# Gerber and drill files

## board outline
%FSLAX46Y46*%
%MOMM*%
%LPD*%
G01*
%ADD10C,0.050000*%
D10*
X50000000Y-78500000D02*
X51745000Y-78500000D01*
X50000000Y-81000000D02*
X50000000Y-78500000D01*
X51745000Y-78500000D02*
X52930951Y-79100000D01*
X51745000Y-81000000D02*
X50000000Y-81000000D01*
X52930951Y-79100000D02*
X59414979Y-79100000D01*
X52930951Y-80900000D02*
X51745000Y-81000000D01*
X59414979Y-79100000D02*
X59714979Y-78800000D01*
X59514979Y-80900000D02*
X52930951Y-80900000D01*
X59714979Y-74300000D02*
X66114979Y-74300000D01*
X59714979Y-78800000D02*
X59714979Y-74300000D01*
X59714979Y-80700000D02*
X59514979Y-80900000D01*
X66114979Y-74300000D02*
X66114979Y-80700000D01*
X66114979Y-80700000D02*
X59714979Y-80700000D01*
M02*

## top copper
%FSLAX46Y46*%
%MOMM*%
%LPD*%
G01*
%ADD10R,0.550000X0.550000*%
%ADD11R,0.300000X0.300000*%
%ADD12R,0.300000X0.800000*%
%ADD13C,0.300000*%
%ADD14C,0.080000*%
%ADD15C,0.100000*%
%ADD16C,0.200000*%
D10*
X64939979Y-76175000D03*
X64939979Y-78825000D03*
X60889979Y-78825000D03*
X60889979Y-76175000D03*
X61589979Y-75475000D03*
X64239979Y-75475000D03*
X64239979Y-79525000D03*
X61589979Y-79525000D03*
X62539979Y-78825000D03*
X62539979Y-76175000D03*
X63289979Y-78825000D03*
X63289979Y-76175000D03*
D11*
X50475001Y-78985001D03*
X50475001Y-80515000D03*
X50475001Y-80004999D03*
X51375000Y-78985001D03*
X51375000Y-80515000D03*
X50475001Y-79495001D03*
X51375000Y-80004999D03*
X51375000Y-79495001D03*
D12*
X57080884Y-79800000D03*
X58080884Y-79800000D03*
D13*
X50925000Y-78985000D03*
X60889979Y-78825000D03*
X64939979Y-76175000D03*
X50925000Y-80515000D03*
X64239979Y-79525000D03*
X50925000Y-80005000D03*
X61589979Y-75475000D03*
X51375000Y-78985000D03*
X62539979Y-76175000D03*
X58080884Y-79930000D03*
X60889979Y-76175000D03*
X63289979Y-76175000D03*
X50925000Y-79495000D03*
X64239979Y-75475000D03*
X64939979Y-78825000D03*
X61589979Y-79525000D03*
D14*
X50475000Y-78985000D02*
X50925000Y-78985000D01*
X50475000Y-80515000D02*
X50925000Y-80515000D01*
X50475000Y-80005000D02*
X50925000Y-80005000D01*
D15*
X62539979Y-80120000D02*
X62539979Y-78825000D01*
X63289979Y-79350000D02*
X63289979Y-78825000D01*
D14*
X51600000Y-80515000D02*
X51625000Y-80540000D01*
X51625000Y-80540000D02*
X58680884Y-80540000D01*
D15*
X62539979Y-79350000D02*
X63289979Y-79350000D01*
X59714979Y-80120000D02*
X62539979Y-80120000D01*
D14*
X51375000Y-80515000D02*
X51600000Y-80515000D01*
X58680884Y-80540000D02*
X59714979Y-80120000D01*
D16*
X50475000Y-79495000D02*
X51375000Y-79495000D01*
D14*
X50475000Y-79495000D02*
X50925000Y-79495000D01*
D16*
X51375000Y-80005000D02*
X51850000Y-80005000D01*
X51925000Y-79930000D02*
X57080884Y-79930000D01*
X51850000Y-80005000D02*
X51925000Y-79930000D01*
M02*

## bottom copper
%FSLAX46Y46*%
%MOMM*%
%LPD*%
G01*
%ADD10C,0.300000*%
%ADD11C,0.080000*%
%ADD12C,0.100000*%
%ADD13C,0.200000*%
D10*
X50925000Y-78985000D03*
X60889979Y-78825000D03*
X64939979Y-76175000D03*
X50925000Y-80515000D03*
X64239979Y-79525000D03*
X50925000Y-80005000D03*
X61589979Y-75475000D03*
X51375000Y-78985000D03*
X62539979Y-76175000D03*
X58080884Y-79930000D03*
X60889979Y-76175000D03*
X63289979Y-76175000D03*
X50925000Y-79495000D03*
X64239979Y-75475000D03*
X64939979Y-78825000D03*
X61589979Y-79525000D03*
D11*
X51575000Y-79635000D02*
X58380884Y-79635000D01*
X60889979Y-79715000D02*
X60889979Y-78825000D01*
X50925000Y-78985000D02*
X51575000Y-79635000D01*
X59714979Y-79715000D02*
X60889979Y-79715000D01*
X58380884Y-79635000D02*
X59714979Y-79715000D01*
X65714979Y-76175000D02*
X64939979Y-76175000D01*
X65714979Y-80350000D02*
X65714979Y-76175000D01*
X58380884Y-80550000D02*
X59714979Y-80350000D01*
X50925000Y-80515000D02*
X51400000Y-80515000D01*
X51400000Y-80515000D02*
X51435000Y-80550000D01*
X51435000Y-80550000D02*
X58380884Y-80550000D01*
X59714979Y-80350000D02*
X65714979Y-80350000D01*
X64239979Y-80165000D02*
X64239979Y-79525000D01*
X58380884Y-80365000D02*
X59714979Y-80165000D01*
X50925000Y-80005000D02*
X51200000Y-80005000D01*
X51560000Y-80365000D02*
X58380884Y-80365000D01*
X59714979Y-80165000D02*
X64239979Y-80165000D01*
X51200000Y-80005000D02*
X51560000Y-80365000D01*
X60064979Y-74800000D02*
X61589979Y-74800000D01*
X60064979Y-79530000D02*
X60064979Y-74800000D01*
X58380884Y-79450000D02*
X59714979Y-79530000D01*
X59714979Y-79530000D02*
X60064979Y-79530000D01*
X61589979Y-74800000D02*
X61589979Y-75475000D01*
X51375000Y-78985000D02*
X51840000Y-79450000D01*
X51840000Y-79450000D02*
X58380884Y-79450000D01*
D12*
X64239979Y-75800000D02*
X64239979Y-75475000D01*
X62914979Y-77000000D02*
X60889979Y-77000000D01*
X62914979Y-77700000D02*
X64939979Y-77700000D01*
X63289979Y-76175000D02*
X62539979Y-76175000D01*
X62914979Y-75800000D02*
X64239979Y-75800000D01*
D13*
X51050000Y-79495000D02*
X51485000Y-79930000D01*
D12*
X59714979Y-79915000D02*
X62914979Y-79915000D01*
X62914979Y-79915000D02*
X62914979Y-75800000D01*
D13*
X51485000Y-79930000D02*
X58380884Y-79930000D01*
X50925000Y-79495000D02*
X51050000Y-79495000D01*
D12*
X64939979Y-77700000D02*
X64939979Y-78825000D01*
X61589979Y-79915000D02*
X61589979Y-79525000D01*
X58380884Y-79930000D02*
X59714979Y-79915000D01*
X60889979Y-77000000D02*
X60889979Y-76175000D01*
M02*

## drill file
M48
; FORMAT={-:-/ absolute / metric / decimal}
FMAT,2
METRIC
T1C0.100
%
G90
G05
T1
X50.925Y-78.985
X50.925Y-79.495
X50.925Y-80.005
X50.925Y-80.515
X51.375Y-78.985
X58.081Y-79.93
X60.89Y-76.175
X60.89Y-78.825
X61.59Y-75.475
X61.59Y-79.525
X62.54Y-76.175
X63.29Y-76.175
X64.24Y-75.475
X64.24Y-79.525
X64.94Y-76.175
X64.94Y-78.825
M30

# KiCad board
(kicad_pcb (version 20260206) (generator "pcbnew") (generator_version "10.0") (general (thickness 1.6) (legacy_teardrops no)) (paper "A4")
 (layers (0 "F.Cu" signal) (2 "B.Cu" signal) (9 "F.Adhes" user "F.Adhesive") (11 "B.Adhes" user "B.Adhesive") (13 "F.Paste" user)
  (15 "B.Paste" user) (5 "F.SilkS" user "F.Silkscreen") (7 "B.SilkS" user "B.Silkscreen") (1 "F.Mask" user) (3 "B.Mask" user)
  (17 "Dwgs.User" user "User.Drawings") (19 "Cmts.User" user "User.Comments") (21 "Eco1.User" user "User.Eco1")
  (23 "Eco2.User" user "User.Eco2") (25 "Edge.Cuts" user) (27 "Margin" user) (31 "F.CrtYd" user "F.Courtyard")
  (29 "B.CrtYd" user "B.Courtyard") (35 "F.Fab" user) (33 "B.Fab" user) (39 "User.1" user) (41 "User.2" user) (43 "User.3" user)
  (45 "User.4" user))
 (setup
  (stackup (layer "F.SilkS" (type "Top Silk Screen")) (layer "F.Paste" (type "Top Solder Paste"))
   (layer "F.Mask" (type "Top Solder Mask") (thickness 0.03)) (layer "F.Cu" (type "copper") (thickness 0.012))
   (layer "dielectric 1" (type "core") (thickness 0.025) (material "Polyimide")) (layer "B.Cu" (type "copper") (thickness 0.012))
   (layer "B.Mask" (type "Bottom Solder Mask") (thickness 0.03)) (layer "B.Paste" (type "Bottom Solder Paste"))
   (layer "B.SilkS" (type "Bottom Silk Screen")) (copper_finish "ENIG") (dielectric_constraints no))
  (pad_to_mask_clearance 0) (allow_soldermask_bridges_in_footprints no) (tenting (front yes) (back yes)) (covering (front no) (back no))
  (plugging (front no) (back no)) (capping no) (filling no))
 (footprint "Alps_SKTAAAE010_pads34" (layer "F.Cu") (at 62.914979 79.9 180)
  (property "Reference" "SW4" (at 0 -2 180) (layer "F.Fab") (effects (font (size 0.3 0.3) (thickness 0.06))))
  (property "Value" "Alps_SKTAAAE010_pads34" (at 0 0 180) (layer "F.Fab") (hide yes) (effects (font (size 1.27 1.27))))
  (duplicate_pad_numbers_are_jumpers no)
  (pad "3" smd rect (at -1.325 0.375 180) (size 0.55 0.55) (layers "F.Cu" "F.Mask" "F.Paste") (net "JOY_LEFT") (solder_mask_margin 0.05)
   (thermal_bridge_angle 45))
  (pad "4" smd rect (at 1.325 0.375 180) (size 0.55 0.55) (layers "F.Cu" "F.Mask" "F.Paste") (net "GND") (solder_mask_margin 0.05)
   (thermal_bridge_angle 45)))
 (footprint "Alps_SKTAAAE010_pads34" (layer "F.Cu") (at 62.914979 75.1)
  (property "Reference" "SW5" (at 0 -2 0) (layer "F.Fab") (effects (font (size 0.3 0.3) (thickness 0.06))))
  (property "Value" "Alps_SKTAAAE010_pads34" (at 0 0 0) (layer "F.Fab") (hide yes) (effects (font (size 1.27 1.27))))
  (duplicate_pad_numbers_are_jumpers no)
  (pad "3" smd rect (at -1.325 0.375) (size 0.55 0.55) (layers "F.Cu" "F.Mask" "F.Paste") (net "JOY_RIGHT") (solder_mask_margin 0.05)
   (thermal_bridge_angle 45))
  (pad "4" smd rect (at 1.325 0.375) (size 0.55 0.55) (layers "F.Cu" "F.Mask" "F.Paste") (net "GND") (solder_mask_margin 0.05)
   (thermal_bridge_angle 45)))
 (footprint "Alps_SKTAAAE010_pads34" (layer "F.Cu") (at 60.514979 77.5 90)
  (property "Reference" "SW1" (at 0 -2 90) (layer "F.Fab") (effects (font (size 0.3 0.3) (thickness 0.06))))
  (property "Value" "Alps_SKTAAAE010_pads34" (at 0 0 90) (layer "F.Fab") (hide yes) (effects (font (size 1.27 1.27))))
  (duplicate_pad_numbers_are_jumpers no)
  (pad "3" smd rect (at -1.325 0.375 90) (size 0.55 0.55) (layers "F.Cu" "F.Mask" "F.Paste") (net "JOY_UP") (solder_mask_margin 0.05)
   (thermal_bridge_angle 45))
  (pad "4" smd rect (at 1.325 0.375 90) (size 0.55 0.55) (layers "F.Cu" "F.Mask" "F.Paste") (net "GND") (solder_mask_margin 0.05)
   (thermal_bridge_angle 45)))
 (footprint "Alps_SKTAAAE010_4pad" (layer "F.Cu") (at 62.914979 77.5 90)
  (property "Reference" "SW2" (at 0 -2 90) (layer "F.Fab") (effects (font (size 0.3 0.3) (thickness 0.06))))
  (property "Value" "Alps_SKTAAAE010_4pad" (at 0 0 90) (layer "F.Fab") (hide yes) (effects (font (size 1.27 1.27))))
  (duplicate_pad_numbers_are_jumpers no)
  (pad "1" smd rect (at -1.325 -0.375 90) (size 0.55 0.55) (layers "F.Cu" "F.Mask" "F.Paste") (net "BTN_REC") (solder_mask_margin 0.05)
   (thermal_bridge_angle 45))
  (pad "2" smd rect (at 1.325 -0.375 90) (size 0.55 0.55) (layers "F.Cu" "F.Mask" "F.Paste") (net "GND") (solder_mask_margin 0.05)
   (thermal_bridge_angle 45))
  (pad "3" smd rect (at -1.325 0.375 90) (size 0.55 0.55) (layers "F.Cu" "F.Mask" "F.Paste") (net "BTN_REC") (solder_mask_margin 0.05)
   (thermal_bridge_angle 45))
  (pad "4" smd rect (at 1.325 0.375 90) (size 0.55 0.55) (layers "F.Cu" "F.Mask" "F.Paste") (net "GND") (solder_mask_margin 0.05)
   (thermal_bridge_angle 45)))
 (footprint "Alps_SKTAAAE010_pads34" (layer "F.Cu") (at 65.314979 77.5 -90)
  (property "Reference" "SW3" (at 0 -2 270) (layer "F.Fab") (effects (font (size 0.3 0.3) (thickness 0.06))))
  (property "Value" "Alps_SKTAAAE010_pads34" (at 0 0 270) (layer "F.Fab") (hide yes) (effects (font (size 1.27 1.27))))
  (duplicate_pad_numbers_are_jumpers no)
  (pad "3" smd rect (at -1.325 0.375 270) (size 0.55 0.55) (layers "F.Cu" "F.Mask" "F.Paste") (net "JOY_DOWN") (solder_mask_margin 0.05)
   (thermal_bridge_angle 45))
  (pad "4" smd rect (at 1.325 0.375 270) (size 0.55 0.55) (layers "F.Cu" "F.Mask" "F.Paste") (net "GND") (solder_mask_margin 0.05)
   (thermal_bridge_angle 45)))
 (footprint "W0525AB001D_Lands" (layer "F.Cu") (at 57.580884 79.93)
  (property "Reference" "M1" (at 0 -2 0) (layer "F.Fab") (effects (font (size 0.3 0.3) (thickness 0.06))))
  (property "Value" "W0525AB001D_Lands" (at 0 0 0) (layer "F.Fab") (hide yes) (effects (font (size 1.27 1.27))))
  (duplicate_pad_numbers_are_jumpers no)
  (pad "1" smd rect (at -0.5 -0.13) (size 0.3 0.8) (layers "F.Cu" "F.Mask") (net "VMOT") (solder_mask_margin 0.05) (thermal_bridge_angle 45))
  (pad "2" smd rect (at 0.5 -0.13) (size 0.3 0.8) (layers "F.Cu" "F.Mask") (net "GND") (solder_mask_margin 0.05) (thermal_bridge_angle 45)))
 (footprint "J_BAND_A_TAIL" (layer "F.Cu") (at 50.9 79.75)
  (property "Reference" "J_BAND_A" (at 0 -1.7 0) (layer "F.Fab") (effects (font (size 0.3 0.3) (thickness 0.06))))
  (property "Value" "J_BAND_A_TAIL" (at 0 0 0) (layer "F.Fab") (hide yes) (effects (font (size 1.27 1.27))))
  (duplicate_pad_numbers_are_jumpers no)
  (pad "1" smd rect (at -0.424999 -0.764999) (size 0.3 0.3) (layers "F.Cu" "F.Mask") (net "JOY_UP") (solder_mask_margin 0.05)
   (thermal_bridge_angle 45))
  (pad "2" smd rect (at -0.424999 0.765) (size 0.3 0.3) (layers "F.Cu" "F.Mask") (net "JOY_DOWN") (solder_mask_margin 0.05)
   (thermal_bridge_angle 45))
  (pad "3" smd rect (at -0.424999 0.254999) (size 0.3 0.3) (layers "F.Cu" "F.Mask") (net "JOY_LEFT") (solder_mask_margin 0.05)
   (thermal_bridge_angle 45))
  (pad "4" smd rect (at 0.475 -0.764999) (size 0.3 0.3) (layers "F.Cu" "F.Mask") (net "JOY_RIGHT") (solder_mask_margin 0.05)
   (thermal_bridge_angle 45))
  (pad "5" smd rect (at 0.475 0.765) (size 0.3 0.3) (layers "F.Cu" "F.Mask") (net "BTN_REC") (solder_mask_margin 0.05)
   (thermal_bridge_angle 45))
  (pad "6" smd rect (at -0.424999 -0.254999) (size 0.3 0.3) (layers "F.Cu" "F.Mask") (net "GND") (solder_mask_margin 0.05)
   (thermal_bridge_angle 45))
  (pad "7" smd rect (at 0.475 0.254999) (size 0.3 0.3) (layers "F.Cu" "F.Mask") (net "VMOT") (solder_mask_margin 0.05)
   (thermal_bridge_angle 45))
  (pad "8" smd rect (at 0.475 -0.254999) (size 0.3 0.3) (layers "F.Cu" "F.Mask") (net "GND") (solder_mask_margin 0.05)
   (thermal_bridge_angle 45)))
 (gr_line (start 50 78.5) (end 51.745 78.5) (stroke (width 0.05) (type default)) (layer "Edge.Cuts"))
 (gr_line (start 50 81) (end 50 78.5) (stroke (width 0.05) (type default)) (layer "Edge.Cuts"))
 (gr_line (start 51.745 78.5) (end 52.930951 79.1) (stroke (width 0.05) (type default)) (layer "Edge.Cuts"))
 (gr_line (start 51.745 81) (end 50 81) (stroke (width 0.05) (type default)) (layer "Edge.Cuts"))
 (gr_line (start 52.930951 79.1) (end 59.414979 79.1) (stroke (width 0.05) (type default)) (layer "Edge.Cuts"))
 (gr_line (start 52.930951 80.9) (end 51.745 81) (stroke (width 0.05) (type default)) (layer "Edge.Cuts"))
 (gr_line (start 59.414979 79.1) (end 59.714979 78.8) (stroke (width 0.05) (type default)) (layer "Edge.Cuts"))
 (gr_line (start 59.514979 80.9) (end 52.930951 80.9) (stroke (width 0.05) (type default)) (layer "Edge.Cuts"))
 (gr_line (start 59.714979 74.3) (end 66.114979 74.3) (stroke (width 0.05) (type default)) (layer "Edge.Cuts"))
 (gr_line (start 59.714979 78.8) (end 59.714979 74.3) (stroke (width 0.05) (type default)) (layer "Edge.Cuts"))
 (gr_line (start 59.714979 80.7) (end 59.514979 80.9) (stroke (width 0.05) (type default)) (layer "Edge.Cuts"))
 (gr_line (start 66.114979 74.3) (end 66.114979 80.7) (stroke (width 0.05) (type default)) (layer "Edge.Cuts"))
 (gr_line (start 66.114979 80.7) (end 59.714979 80.7) (stroke (width 0.05) (type default)) (layer "Edge.Cuts"))
 (segment (start 50.475 78.985) (end 50.925 78.985) (width 0.08) (layer "F.Cu") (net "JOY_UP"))
 (via (at 60.889979 78.825) (size 0.3) (drill 0.1) (layers "F.Cu" "B.Cu") (tenting (front yes) (back yes)) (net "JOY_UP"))
 (via (at 50.925 78.985) (size 0.3) (drill 0.1) (layers "F.Cu" "B.Cu") (tenting (front yes) (back yes)) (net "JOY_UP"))
 (segment (start 58.380884 79.635) (end 59.714979 79.715) (width 0.08) (layer "B.Cu") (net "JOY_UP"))
 (segment (start 51.575 79.635) (end 58.380884 79.635) (width 0.08) (layer "B.Cu") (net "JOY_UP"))
 (segment (start 59.714979 79.715) (end 60.889979 79.715) (width 0.08) (layer "B.Cu") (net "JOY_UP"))
 (segment (start 50.925 78.985) (end 51.575 79.635) (width 0.08) (layer "B.Cu") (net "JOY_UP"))
 (segment (start 60.889979 79.715) (end 60.889979 78.825) (width 0.08) (layer "B.Cu") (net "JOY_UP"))
 (segment (start 50.475 80.515) (end 50.925 80.515) (width 0.08) (layer "F.Cu") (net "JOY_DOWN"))
 (via (at 64.939979 76.175) (size 0.3) (drill 0.1) (layers "F.Cu" "B.Cu") (tenting (front yes) (back yes)) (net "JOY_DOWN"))
 (via (at 50.925 80.515) (size 0.3) (drill 0.1) (layers "F.Cu" "B.Cu") (tenting (front yes) (back yes)) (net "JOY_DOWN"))
 (segment (start 58.380884 80.55) (end 59.714979 80.35) (width 0.08) (layer "B.Cu") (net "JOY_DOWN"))
 (segment (start 65.714979 76.175) (end 64.939979 76.175) (width 0.08) (layer "B.Cu") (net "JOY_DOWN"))
 (segment (start 51.4 80.515) (end 51.435 80.55) (width 0.08) (layer "B.Cu") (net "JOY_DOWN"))
 (segment (start 51.435 80.55) (end 58.380884 80.55) (width 0.08) (layer "B.Cu") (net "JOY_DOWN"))
 (segment (start 59.714979 80.35) (end 65.714979 80.35) (width 0.08) (layer "B.Cu") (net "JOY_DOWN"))
 (segment (start 50.925 80.515) (end 51.4 80.515) (width 0.08) (layer "B.Cu") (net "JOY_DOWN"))
 (segment (start 65.714979 80.35) (end 65.714979 76.175) (width 0.08) (layer "B.Cu") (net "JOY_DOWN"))
 (segment (start 50.475 80.005) (end 50.925 80.005) (width 0.08) (layer "F.Cu") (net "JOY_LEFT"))
 (via (at 50.925 80.005) (size 0.3) (drill 0.1) (layers "F.Cu" "B.Cu") (tenting (front yes) (back yes)) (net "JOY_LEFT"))
 (via (at 64.239979 79.525) (size 0.3) (drill 0.1) (layers "F.Cu" "B.Cu") (tenting (front yes) (back yes)) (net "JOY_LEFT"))
 (segment (start 50.925 80.005) (end 51.2 80.005) (width 0.08) (layer "B.Cu") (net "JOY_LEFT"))
 (segment (start 51.2 80.005) (end 51.56 80.365) (width 0.08) (layer "B.Cu") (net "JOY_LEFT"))
 (segment (start 59.714979 80.165) (end 64.239979 80.165) (width 0.08) (layer "B.Cu") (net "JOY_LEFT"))
 (segment (start 58.380884 80.365) (end 59.714979 80.165) (width 0.08) (layer "B.Cu") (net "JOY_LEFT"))
 (segment (start 51.56 80.365) (end 58.380884 80.365) (width 0.08) (layer "B.Cu") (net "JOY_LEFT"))
 (segment (start 64.239979 80.165) (end 64.239979 79.525) (width 0.08) (layer "B.Cu") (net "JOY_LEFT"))
 (via (at 51.375 78.985) (size 0.3) (drill 0.1) (layers "F.Cu" "B.Cu") (tenting (front yes) (back yes)) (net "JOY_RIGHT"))
 (via (at 61.589979 75.475) (size 0.3) (drill 0.1) (layers "F.Cu" "B.Cu") (tenting (front yes) (back yes)) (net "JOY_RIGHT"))
 (segment (start 59.714979 79.53) (end 60.064979 79.53) (width 0.08) (layer "B.Cu") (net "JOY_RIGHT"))
 (segment (start 58.380884 79.45) (end 59.714979 79.53) (width 0.08) (layer "B.Cu") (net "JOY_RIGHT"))
 (segment (start 60.064979 79.53) (end 60.064979 74.8) (width 0.08) (layer "B.Cu") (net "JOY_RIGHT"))
 (segment (start 60.064979 74.8) (end 61.589979 74.8) (width 0.08) (layer "B.Cu") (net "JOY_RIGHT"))
 (segment (start 51.84 79.45) (end 58.380884 79.45) (width 0.08) (layer "B.Cu") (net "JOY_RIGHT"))
 (segment (start 51.375 78.985) (end 51.84 79.45) (width 0.08) (layer "B.Cu") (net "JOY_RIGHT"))
 (segment (start 61.589979 74.8) (end 61.589979 75.475) (width 0.08) (layer "B.Cu") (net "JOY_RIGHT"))
 (segment (start 59.714979 80.12) (end 62.539979 80.12) (width 0.1) (layer "F.Cu") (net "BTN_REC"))
 (segment (start 51.375 80.515) (end 51.6 80.515) (width 0.08) (layer "F.Cu") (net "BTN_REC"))
 (segment (start 51.625 80.54) (end 58.680884 80.54) (width 0.08) (layer "F.Cu") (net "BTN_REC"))
 (segment (start 62.539979 79.35) (end 63.289979 79.35) (width 0.1) (layer "F.Cu") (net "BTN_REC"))
 (segment (start 51.6 80.515) (end 51.625 80.54) (width 0.08) (layer "F.Cu") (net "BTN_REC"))
 (segment (start 63.289979 79.35) (end 63.289979 78.825) (width 0.1) (layer "F.Cu") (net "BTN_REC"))
 (segment (start 62.539979 80.12) (end 62.539979 78.825) (width 0.1) (layer "F.Cu") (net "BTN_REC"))
 (segment (start 58.680884 80.54) (end 59.714979 80.12) (width 0.08) (layer "F.Cu") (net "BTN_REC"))
 (segment (start 50.475 79.495) (end 50.925 79.495) (width 0.08) (layer "F.Cu") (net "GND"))
 (segment (start 50.475 79.495) (end 51.375 79.495) (width 0.2) (layer "F.Cu") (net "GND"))
 (via (at 62.539979 76.175) (size 0.3) (drill 0.1) (layers "F.Cu" "B.Cu") (tenting (front yes) (back yes)) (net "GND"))
 (via (at 64.939979 78.825) (size 0.3) (drill 0.1) (layers "F.Cu" "B.Cu") (tenting (front yes) (back yes)) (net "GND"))
 (via (at 60.889979 76.175) (size 0.3) (drill 0.1) (layers "F.Cu" "B.Cu") (tenting (front yes) (back yes)) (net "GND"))
 (via (at 63.289979 76.175) (size 0.3) (drill 0.1) (layers "F.Cu" "B.Cu") (tenting (front yes) (back yes)) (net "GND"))
 (via (at 58.080884 79.93) (size 0.3) (drill 0.1) (layers "F.Cu" "B.Cu") (tenting (front yes) (back yes)) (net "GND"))
 (via (at 61.589979 79.525) (size 0.3) (drill 0.1) (layers "F.Cu" "B.Cu") (tenting (front yes) (back yes)) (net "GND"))
 (via (at 50.925 79.495) (size 0.3) (drill 0.1) (layers "F.Cu" "B.Cu") (tenting (front yes) (back yes)) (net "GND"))
 (via (at 64.239979 75.475) (size 0.3) (drill 0.1) (layers "F.Cu" "B.Cu") (tenting (front yes) (back yes)) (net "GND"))
 (segment (start 51.05 79.495) (end 51.485 79.93) (width 0.2) (layer "B.Cu") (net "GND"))
 (segment (start 51.485 79.93) (end 58.380884 79.93) (width 0.2) (layer "B.Cu") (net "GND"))
 (segment (start 64.239979 75.8) (end 64.239979 75.475) (width 0.1) (layer "B.Cu") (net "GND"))
 (segment (start 62.914979 75.8) (end 64.239979 75.8) (width 0.1) (layer "B.Cu") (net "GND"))
 (segment (start 59.714979 79.915) (end 62.914979 79.915) (width 0.1) (layer "B.Cu") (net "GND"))
 (segment (start 62.914979 79.915) (end 62.914979 75.8) (width 0.1) (layer "B.Cu") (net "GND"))
 (segment (start 60.889979 77) (end 60.889979 76.175) (width 0.1) (layer "B.Cu") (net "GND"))
 (segment (start 50.925 79.495) (end 51.05 79.495) (width 0.2) (layer "B.Cu") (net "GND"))
 (segment (start 62.914979 77.7) (end 64.939979 77.7) (width 0.1) (layer "B.Cu") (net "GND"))
 (segment (start 61.589979 79.915) (end 61.589979 79.525) (width 0.1) (layer "B.Cu") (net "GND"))
 (segment (start 63.289979 76.175) (end 62.539979 76.175) (width 0.1) (layer "B.Cu") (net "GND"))
 (segment (start 64.939979 77.7) (end 64.939979 78.825) (width 0.1) (layer "B.Cu") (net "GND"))
 (segment (start 62.914979 77) (end 60.889979 77) (width 0.1) (layer "B.Cu") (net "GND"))
 (segment (start 58.380884 79.93) (end 59.714979 79.915) (width 0.1) (layer "B.Cu") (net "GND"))
 (segment (start 51.85 80.005) (end 51.925 79.93) (width 0.2) (layer "F.Cu") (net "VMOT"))
 (segment (start 51.925 79.93) (end 57.080884 79.93) (width 0.2) (layer "F.Cu") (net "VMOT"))
 (segment (start 51.375 80.005) (end 51.85 80.005) (width 0.2) (layer "F.Cu") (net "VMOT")))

